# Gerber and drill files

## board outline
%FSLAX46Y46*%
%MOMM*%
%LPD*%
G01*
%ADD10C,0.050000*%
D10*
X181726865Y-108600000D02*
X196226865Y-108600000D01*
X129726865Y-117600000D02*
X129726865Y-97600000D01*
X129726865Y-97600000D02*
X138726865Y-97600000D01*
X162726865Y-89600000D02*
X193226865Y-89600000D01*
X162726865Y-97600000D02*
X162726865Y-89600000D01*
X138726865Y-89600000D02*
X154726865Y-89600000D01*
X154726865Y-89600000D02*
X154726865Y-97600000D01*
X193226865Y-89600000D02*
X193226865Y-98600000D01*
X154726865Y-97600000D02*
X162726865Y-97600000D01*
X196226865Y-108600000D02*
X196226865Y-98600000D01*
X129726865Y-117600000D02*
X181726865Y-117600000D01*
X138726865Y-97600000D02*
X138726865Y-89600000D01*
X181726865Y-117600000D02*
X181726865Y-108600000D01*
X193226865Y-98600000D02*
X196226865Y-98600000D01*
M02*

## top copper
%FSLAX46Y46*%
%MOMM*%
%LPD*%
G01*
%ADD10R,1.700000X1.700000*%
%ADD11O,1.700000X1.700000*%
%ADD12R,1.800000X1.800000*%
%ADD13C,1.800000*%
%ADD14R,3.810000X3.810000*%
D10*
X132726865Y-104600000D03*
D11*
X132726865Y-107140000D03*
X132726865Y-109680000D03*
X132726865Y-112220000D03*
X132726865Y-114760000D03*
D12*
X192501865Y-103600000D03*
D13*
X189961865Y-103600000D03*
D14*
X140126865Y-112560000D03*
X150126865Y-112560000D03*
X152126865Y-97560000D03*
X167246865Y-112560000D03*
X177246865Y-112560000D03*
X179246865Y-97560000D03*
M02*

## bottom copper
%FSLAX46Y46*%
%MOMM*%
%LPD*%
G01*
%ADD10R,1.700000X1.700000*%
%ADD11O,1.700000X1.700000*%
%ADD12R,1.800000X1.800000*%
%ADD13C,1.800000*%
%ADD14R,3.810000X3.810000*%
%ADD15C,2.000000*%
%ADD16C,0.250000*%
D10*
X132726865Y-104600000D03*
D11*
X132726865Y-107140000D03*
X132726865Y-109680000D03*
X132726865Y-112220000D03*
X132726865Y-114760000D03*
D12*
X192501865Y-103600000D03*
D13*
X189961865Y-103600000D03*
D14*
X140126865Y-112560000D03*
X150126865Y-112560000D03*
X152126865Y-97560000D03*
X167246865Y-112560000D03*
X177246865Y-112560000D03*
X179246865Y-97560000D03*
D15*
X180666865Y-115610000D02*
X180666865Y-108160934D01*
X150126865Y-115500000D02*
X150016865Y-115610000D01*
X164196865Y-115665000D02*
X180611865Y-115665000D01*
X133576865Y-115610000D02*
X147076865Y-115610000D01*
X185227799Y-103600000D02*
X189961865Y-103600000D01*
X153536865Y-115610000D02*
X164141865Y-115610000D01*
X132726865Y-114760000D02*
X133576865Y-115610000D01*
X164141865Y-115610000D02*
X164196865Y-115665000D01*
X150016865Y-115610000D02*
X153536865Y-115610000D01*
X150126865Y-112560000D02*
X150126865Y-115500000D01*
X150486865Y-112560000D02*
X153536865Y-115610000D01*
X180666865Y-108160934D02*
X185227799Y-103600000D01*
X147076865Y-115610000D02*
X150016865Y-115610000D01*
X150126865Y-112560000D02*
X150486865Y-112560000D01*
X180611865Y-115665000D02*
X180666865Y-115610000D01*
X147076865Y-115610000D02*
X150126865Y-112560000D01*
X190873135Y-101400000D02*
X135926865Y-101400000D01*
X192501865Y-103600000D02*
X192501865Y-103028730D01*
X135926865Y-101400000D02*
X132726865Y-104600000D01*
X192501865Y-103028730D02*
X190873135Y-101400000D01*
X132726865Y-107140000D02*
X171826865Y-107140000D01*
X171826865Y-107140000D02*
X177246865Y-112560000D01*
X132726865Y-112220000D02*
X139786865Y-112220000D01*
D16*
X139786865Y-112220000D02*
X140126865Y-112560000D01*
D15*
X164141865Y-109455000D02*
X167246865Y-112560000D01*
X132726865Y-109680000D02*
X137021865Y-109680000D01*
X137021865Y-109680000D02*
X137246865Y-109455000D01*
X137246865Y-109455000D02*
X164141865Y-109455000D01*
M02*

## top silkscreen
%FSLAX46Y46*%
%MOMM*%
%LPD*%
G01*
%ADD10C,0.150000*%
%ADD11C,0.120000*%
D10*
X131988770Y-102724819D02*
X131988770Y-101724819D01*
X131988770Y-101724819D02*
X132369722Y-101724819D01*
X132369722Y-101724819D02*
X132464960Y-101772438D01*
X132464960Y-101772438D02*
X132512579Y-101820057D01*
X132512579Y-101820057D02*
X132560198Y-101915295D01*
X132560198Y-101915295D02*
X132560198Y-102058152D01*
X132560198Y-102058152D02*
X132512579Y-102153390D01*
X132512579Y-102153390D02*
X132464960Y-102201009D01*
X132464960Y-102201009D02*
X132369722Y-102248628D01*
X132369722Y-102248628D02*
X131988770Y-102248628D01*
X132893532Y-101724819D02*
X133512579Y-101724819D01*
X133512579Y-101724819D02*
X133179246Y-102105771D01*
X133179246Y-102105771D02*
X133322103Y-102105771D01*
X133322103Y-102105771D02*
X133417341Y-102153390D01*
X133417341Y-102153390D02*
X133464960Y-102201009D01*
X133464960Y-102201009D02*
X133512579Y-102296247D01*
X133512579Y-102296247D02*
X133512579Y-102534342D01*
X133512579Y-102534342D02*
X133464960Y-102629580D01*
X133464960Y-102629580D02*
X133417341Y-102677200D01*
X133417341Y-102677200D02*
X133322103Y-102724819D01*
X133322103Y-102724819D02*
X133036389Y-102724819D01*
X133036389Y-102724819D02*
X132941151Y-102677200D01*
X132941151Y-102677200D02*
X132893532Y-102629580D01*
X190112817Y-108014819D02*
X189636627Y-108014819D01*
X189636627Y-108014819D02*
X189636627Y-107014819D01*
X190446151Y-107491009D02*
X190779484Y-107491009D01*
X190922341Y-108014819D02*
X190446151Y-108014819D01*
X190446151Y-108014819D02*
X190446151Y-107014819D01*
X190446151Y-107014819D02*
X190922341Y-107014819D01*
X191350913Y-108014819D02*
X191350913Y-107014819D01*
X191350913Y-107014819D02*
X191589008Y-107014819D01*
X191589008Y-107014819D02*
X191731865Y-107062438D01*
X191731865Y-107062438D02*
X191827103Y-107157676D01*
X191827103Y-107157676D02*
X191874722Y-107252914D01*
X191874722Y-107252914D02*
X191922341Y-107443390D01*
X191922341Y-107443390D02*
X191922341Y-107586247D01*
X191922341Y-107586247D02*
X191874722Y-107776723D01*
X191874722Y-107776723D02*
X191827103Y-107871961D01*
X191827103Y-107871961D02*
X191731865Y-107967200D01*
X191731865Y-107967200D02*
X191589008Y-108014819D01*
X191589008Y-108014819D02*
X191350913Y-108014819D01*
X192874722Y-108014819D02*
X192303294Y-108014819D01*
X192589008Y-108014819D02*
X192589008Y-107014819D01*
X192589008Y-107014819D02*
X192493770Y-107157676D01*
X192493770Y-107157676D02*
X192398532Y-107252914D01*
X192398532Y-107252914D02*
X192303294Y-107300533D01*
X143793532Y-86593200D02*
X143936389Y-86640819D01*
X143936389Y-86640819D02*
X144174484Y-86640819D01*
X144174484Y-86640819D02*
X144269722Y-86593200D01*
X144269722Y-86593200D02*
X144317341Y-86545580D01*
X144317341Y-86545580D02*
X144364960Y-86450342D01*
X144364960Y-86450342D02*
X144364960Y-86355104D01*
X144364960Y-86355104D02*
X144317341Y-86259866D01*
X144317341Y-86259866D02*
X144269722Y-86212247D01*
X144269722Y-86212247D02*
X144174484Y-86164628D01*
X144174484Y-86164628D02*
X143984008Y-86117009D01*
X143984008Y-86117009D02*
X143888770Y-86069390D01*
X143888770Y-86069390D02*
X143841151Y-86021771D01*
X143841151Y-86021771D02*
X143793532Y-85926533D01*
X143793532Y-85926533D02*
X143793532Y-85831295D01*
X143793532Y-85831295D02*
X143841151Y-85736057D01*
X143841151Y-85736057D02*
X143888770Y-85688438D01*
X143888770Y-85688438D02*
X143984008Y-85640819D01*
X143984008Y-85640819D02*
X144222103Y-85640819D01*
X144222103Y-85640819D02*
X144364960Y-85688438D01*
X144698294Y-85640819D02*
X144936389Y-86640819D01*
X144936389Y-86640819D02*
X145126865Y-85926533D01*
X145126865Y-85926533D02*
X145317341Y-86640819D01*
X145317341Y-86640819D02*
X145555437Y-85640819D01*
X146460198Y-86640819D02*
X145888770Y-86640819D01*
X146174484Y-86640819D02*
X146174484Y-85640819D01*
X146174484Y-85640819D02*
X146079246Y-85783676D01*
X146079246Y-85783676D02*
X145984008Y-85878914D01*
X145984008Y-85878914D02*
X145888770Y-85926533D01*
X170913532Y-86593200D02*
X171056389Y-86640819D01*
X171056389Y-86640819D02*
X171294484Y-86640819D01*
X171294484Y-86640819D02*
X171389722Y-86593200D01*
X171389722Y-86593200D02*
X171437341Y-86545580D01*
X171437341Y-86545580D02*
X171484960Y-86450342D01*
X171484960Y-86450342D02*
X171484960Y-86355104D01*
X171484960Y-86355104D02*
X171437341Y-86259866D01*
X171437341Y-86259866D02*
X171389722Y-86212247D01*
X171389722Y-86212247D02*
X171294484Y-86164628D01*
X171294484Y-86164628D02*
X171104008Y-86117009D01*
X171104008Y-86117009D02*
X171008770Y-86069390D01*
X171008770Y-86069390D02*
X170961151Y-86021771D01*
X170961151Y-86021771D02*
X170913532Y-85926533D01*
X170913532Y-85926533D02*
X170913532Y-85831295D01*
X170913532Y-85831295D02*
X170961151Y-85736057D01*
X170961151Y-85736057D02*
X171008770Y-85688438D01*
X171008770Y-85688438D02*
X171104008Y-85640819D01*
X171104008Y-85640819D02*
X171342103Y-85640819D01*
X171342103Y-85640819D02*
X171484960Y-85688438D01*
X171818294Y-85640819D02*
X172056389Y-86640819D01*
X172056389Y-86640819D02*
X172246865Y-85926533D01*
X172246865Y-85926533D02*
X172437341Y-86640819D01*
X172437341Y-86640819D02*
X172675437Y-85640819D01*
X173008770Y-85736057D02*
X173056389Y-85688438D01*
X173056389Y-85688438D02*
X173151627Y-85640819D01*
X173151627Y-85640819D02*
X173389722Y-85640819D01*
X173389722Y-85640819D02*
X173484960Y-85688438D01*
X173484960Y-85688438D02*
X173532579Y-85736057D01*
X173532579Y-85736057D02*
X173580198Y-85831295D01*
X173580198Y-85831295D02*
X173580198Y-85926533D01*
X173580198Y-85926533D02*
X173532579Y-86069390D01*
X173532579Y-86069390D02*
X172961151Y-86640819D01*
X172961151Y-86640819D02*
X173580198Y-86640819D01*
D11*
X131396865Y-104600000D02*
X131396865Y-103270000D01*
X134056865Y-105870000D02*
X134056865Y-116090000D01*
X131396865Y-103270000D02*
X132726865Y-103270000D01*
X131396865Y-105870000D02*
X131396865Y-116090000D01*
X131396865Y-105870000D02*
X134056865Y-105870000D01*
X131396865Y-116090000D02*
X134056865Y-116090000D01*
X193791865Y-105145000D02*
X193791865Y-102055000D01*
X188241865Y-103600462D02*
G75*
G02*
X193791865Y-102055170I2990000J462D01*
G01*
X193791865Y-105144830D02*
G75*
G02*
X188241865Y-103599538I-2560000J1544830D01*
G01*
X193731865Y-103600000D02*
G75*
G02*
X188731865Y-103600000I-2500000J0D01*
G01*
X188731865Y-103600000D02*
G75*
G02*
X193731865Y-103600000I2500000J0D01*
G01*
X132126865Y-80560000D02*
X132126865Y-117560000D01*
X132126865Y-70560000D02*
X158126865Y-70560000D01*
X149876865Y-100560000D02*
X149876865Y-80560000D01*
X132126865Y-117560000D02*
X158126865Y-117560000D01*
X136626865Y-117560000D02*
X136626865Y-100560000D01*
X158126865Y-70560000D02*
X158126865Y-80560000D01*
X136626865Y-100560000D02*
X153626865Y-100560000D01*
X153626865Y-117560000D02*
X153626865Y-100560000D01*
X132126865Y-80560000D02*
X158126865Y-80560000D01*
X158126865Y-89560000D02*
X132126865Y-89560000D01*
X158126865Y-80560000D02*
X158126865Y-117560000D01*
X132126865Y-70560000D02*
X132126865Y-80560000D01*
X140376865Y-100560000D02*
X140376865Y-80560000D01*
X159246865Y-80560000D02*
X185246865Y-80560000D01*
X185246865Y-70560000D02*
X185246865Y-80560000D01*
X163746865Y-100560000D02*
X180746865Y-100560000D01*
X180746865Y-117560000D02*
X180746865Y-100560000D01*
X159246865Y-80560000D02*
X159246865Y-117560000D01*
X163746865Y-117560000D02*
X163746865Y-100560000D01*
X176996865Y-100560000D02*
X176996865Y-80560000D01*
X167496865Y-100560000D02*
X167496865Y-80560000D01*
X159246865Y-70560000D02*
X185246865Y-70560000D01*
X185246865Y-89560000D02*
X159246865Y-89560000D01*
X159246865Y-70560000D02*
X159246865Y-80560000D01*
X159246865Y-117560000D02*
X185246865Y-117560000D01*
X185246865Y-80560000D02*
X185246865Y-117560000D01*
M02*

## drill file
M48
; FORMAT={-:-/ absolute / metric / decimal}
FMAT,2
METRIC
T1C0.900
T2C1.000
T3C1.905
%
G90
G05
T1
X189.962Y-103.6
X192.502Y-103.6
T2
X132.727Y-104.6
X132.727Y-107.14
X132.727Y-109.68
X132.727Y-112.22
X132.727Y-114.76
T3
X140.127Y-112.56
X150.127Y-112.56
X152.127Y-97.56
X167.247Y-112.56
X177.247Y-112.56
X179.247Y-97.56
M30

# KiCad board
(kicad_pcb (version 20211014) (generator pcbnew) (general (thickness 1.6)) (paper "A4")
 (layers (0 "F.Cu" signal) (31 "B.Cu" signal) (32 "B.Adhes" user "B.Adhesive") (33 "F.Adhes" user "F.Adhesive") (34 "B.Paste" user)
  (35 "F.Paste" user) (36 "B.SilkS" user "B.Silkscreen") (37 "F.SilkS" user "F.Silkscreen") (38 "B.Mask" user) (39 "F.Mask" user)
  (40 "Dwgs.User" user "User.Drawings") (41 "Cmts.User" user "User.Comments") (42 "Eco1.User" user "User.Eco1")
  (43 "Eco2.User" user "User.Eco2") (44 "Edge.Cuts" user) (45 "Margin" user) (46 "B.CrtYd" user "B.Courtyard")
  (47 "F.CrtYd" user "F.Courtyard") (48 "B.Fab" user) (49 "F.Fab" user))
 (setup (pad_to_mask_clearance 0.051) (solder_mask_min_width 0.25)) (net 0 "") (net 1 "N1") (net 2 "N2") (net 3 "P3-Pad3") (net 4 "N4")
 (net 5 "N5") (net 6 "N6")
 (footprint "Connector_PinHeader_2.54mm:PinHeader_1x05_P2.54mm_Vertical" (layer "F.Cu") (at 132.726865 104.6)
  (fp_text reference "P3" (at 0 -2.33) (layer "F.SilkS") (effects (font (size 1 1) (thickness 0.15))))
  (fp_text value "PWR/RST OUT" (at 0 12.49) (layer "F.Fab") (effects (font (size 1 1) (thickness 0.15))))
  (fp_line (start -1.33 0) (end -1.33 -1.33) (layer "F.SilkS") (width 0.12))
  (fp_line (start 1.33 1.27) (end 1.33 11.49) (layer "F.SilkS") (width 0.12))
  (fp_line (start -1.33 -1.33) (end 0 -1.33) (layer "F.SilkS") (width 0.12))
  (fp_line (start -1.33 1.27) (end -1.33 11.49) (layer "F.SilkS") (width 0.12))
  (fp_line (start -1.33 1.27) (end 1.33 1.27) (layer "F.SilkS") (width 0.12))
  (fp_line (start -1.33 11.49) (end 1.33 11.49) (layer "F.SilkS") (width 0.12))
  (pad "1" thru_hole rect (at 0 0) (size 1.7 1.7) (drill 1) (layers *.Cu *.Mask) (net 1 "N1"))
  (pad "2" thru_hole oval (at 0 2.54) (size 1.7 1.7) (drill 1) (layers *.Cu *.Mask) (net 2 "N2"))
  (pad "3" thru_hole oval (at 0 5.08) (size 1.7 1.7) (drill 1) (layers *.Cu *.Mask) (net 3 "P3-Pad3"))
  (pad "4" thru_hole oval (at 0 7.62) (size 1.7 1.7) (drill 1) (layers *.Cu *.Mask) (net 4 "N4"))
  (pad "5" thru_hole oval (at 0 10.16) (size 1.7 1.7) (drill 1) (layers *.Cu *.Mask) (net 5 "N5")))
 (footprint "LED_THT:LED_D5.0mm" (layer "F.Cu") (at 192.501865 103.6 180)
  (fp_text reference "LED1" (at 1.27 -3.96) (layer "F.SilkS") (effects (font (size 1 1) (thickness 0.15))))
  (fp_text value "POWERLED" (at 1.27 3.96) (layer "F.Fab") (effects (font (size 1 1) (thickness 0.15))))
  (fp_line (start -1.29 -1.545) (end -1.29 1.545) (layer "F.SilkS") (width 0.12))
  (fp_arc (start 4.26 -0.000462) (mid 2.072002 2.880433) (end -1.29 1.54483) (layer "F.SilkS") (width 0.12))
  (fp_arc (start -1.29 -1.54483) (mid 2.072002 -2.880433) (end 4.26 0.000462) (layer "F.SilkS") (width 0.12))
  (fp_circle (center 1.27 0) (end 3.77 0) (layer "F.SilkS") (width 0.12) (fill none))
  (pad "1" thru_hole rect (at 0 0 180) (size 1.8 1.8) (drill 0.9) (layers *.Cu *.Mask) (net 1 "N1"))
  (pad "2" thru_hole circle (at 2.54 0 180) (size 1.8 1.8) (drill 0.9) (layers *.Cu *.Mask) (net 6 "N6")))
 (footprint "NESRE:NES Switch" (layer "F.Cu") (at 145.126865 94.06)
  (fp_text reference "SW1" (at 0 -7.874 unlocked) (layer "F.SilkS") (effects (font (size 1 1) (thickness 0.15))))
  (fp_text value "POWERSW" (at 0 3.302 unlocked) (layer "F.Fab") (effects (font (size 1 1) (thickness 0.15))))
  (fp_line (start -13 -13.5) (end -13 23.5) (layer "F.SilkS") (width 0.12))
  (fp_line (start -13 -23.5) (end 13 -23.5) (layer "F.SilkS") (width 0.12))
  (fp_line (start 4.75 6.5) (end 4.75 -13.5) (layer "F.SilkS") (width 0.12))
  (fp_line (start -13 23.5) (end 13 23.5) (layer "F.SilkS") (width 0.12))
  (fp_line (start -8.5 23.5) (end -8.5 6.5) (layer "F.SilkS") (width 0.12))
  (fp_line (start 13 -23.5) (end 13 -13.5) (layer "F.SilkS") (width 0.12))
  (fp_line (start -8.5 6.5) (end 8.5 6.5) (layer "F.SilkS") (width 0.12))
  (fp_line (start 8.5 23.5) (end 8.5 6.5) (layer "F.SilkS") (width 0.12))
  (fp_line (start -13 -13.5) (end 13 -13.5) (layer "F.SilkS") (width 0.12))
  (fp_line (start 13 -4.5) (end -13 -4.5) (layer "F.SilkS") (width 0.12))
  (fp_line (start 13 -13.5) (end 13 23.5) (layer "F.SilkS") (width 0.12))
  (fp_line (start -13 -23.5) (end -13 -13.5) (layer "F.SilkS") (width 0.12))
  (fp_line (start -4.75 6.5) (end -4.75 -13.5) (layer "F.SilkS") (width 0.12))
  (pad "1" thru_hole rect (at -5 18.5) (size 3.81 3.81) (drill 1.905) (layers *.Cu *.Mask) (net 4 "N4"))
  (pad "2" thru_hole rect (at 5 18.5) (size 3.81 3.81) (drill 1.905) (layers *.Cu *.Mask) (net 5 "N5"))
  (pad "NC" thru_hole rect (at 7 3.5) (size 3.81 3.81) (drill 1.905) (layers *.Cu *.Mask)))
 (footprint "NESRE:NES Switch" (layer "F.Cu") (at 172.246865 94.06)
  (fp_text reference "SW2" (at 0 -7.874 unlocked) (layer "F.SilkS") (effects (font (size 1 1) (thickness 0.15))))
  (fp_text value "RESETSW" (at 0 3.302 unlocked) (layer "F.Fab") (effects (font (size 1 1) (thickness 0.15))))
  (fp_line (start -13 -13.5) (end 13 -13.5) (layer "F.SilkS") (width 0.12))
  (fp_line (start 13 -23.5) (end 13 -13.5) (layer "F.SilkS") (width 0.12))
  (fp_line (start -8.5 6.5) (end 8.5 6.5) (layer "F.SilkS") (width 0.12))
  (fp_line (start 8.5 23.5) (end 8.5 6.5) (layer "F.SilkS") (width 0.12))
  (fp_line (start -13 -13.5) (end -13 23.5) (layer "F.SilkS") (width 0.12))
  (fp_line (start -8.5 23.5) (end -8.5 6.5) (layer "F.SilkS") (width 0.12))
  (fp_line (start 4.75 6.5) (end 4.75 -13.5) (layer "F.SilkS") (width 0.12))
  (fp_line (start -4.75 6.5) (end -4.75 -13.5) (layer "F.SilkS") (width 0.12))
  (fp_line (start -13 -23.5) (end 13 -23.5) (layer "F.SilkS") (width 0.12))
  (fp_line (start 13 -4.5) (end -13 -4.5) (layer "F.SilkS") (width 0.12))
  (fp_line (start -13 -23.5) (end -13 -13.5) (layer "F.SilkS") (width 0.12))
  (fp_line (start -13 23.5) (end 13 23.5) (layer "F.SilkS") (width 0.12))
  (fp_line (start 13 -13.5) (end 13 23.5) (layer "F.SilkS") (width 0.12))
  (pad "1" thru_hole rect (at -5 18.5) (size 3.81 3.81) (drill 1.905) (layers *.Cu *.Mask) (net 3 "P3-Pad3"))
  (pad "2" thru_hole rect (at 5 18.5) (size 3.81 3.81) (drill 1.905) (layers *.Cu *.Mask) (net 2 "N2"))
  (pad "NC" thru_hole rect (at 7 3.5) (size 3.81 3.81) (drill 1.905) (layers *.Cu *.Mask)))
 (gr_line (start 181.726865 108.6) (end 196.226865 108.6) (layer "Edge.Cuts") (width 0.05))
 (gr_line (start 129.726865 117.6) (end 129.726865 97.6) (layer "Edge.Cuts") (width 0.05))
 (gr_line (start 129.726865 97.6) (end 138.726865 97.6) (layer "Edge.Cuts") (width 0.05))
 (gr_line (start 162.726865 89.6) (end 193.226865 89.6) (layer "Edge.Cuts") (width 0.05))
 (gr_line (start 162.726865 97.6) (end 162.726865 89.6) (layer "Edge.Cuts") (width 0.05))
 (gr_line (start 138.726865 89.6) (end 154.726865 89.6) (layer "Edge.Cuts") (width 0.05))
 (gr_line (start 154.726865 89.6) (end 154.726865 97.6) (layer "Edge.Cuts") (width 0.05))
 (gr_line (start 193.226865 89.6) (end 193.226865 98.6) (layer "Edge.Cuts") (width 0.05))
 (gr_line (start 154.726865 97.6) (end 162.726865 97.6) (layer "Edge.Cuts") (width 0.05))
 (gr_line (start 196.226865 108.6) (end 196.226865 98.6) (layer "Edge.Cuts") (width 0.05))
 (gr_line (start 129.726865 117.6) (end 181.726865 117.6) (layer "Edge.Cuts") (width 0.05))
 (gr_line (start 138.726865 97.6) (end 138.726865 89.6) (layer "Edge.Cuts") (width 0.05))
 (gr_line (start 181.726865 117.6) (end 181.726865 108.6) (layer "Edge.Cuts") (width 0.05))
 (gr_line (start 193.226865 98.6) (end 196.226865 98.6) (layer "Edge.Cuts") (width 0.05))
 (segment (start 180.666865 115.61) (end 180.666865 108.160934) (width 2) (layer "B.Cu") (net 5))
 (segment (start 150.126865 115.5) (end 150.016865 115.61) (width 2) (layer "B.Cu") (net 5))
 (segment (start 164.196865 115.665) (end 180.611865 115.665) (width 2) (layer "B.Cu") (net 5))
 (segment (start 133.576865 115.61) (end 147.076865 115.61) (width 2) (layer "B.Cu") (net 5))
 (segment (start 185.227799 103.6) (end 189.961865 103.6) (width 2) (layer "B.Cu") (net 5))
 (segment (start 153.536865 115.61) (end 164.141865 115.61) (width 2) (layer "B.Cu") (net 5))
 (segment (start 132.726865 114.76) (end 133.576865 115.61) (width 2) (layer "B.Cu") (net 5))
 (segment (start 164.141865 115.61) (end 164.196865 115.665) (width 2) (layer "B.Cu") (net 5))
 (segment (start 150.016865 115.61) (end 153.536865 115.61) (width 2) (layer "B.Cu") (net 5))
 (segment (start 150.126865 112.56) (end 150.126865 115.5) (width 2) (layer "B.Cu") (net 5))
 (segment (start 150.486865 112.56) (end 153.536865 115.61) (width 2) (layer "B.Cu") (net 5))
 (segment (start 180.666865 108.160934) (end 185.227799 103.6) (width 2) (layer "B.Cu") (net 5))
 (segment (start 147.076865 115.61) (end 150.016865 115.61) (width 2) (layer "B.Cu") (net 5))
 (segment (start 150.126865 112.56) (end 150.486865 112.56) (width 2) (layer "B.Cu") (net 5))
 (segment (start 180.611865 115.665) (end 180.666865 115.61) (width 2) (layer "B.Cu") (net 5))
 (segment (start 147.076865 115.61) (end 150.126865 112.56) (width 2) (layer "B.Cu") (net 5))
 (segment (start 190.873135 101.4) (end 135.926865 101.4) (width 2) (layer "B.Cu") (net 1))
 (segment (start 192.501865 103.6) (end 192.501865 103.02873) (width 2) (layer "B.Cu") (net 1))
 (segment (start 135.926865 101.4) (end 132.726865 104.6) (width 2) (layer "B.Cu") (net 1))
 (segment (start 192.501865 103.02873) (end 190.873135 101.4) (width 2) (layer "B.Cu") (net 1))
 (segment (start 132.726865 107.14) (end 171.826865 107.14) (width 2) (layer "B.Cu") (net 2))
 (segment (start 171.826865 107.14) (end 177.246865 112.56) (width 2) (layer "B.Cu") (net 2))
 (segment (start 132.726865 112.22) (end 139.786865 112.22) (width 2) (layer "B.Cu") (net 4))
 (segment (start 139.786865 112.22) (end 140.126865 112.56) (width 0.25) (layer "B.Cu") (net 4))
 (segment (start 164.141865 109.455) (end 167.246865 112.56) (width 2) (layer "B.Cu") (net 3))
 (segment (start 132.726865 109.68) (end 137.021865 109.68) (width 2) (layer "B.Cu") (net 3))
 (segment (start 137.021865 109.68) (end 137.246865 109.455) (width 2) (layer "B.Cu") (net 3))
 (segment (start 137.246865 109.455) (end 164.141865 109.455) (width 2) (layer "B.Cu") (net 3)))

